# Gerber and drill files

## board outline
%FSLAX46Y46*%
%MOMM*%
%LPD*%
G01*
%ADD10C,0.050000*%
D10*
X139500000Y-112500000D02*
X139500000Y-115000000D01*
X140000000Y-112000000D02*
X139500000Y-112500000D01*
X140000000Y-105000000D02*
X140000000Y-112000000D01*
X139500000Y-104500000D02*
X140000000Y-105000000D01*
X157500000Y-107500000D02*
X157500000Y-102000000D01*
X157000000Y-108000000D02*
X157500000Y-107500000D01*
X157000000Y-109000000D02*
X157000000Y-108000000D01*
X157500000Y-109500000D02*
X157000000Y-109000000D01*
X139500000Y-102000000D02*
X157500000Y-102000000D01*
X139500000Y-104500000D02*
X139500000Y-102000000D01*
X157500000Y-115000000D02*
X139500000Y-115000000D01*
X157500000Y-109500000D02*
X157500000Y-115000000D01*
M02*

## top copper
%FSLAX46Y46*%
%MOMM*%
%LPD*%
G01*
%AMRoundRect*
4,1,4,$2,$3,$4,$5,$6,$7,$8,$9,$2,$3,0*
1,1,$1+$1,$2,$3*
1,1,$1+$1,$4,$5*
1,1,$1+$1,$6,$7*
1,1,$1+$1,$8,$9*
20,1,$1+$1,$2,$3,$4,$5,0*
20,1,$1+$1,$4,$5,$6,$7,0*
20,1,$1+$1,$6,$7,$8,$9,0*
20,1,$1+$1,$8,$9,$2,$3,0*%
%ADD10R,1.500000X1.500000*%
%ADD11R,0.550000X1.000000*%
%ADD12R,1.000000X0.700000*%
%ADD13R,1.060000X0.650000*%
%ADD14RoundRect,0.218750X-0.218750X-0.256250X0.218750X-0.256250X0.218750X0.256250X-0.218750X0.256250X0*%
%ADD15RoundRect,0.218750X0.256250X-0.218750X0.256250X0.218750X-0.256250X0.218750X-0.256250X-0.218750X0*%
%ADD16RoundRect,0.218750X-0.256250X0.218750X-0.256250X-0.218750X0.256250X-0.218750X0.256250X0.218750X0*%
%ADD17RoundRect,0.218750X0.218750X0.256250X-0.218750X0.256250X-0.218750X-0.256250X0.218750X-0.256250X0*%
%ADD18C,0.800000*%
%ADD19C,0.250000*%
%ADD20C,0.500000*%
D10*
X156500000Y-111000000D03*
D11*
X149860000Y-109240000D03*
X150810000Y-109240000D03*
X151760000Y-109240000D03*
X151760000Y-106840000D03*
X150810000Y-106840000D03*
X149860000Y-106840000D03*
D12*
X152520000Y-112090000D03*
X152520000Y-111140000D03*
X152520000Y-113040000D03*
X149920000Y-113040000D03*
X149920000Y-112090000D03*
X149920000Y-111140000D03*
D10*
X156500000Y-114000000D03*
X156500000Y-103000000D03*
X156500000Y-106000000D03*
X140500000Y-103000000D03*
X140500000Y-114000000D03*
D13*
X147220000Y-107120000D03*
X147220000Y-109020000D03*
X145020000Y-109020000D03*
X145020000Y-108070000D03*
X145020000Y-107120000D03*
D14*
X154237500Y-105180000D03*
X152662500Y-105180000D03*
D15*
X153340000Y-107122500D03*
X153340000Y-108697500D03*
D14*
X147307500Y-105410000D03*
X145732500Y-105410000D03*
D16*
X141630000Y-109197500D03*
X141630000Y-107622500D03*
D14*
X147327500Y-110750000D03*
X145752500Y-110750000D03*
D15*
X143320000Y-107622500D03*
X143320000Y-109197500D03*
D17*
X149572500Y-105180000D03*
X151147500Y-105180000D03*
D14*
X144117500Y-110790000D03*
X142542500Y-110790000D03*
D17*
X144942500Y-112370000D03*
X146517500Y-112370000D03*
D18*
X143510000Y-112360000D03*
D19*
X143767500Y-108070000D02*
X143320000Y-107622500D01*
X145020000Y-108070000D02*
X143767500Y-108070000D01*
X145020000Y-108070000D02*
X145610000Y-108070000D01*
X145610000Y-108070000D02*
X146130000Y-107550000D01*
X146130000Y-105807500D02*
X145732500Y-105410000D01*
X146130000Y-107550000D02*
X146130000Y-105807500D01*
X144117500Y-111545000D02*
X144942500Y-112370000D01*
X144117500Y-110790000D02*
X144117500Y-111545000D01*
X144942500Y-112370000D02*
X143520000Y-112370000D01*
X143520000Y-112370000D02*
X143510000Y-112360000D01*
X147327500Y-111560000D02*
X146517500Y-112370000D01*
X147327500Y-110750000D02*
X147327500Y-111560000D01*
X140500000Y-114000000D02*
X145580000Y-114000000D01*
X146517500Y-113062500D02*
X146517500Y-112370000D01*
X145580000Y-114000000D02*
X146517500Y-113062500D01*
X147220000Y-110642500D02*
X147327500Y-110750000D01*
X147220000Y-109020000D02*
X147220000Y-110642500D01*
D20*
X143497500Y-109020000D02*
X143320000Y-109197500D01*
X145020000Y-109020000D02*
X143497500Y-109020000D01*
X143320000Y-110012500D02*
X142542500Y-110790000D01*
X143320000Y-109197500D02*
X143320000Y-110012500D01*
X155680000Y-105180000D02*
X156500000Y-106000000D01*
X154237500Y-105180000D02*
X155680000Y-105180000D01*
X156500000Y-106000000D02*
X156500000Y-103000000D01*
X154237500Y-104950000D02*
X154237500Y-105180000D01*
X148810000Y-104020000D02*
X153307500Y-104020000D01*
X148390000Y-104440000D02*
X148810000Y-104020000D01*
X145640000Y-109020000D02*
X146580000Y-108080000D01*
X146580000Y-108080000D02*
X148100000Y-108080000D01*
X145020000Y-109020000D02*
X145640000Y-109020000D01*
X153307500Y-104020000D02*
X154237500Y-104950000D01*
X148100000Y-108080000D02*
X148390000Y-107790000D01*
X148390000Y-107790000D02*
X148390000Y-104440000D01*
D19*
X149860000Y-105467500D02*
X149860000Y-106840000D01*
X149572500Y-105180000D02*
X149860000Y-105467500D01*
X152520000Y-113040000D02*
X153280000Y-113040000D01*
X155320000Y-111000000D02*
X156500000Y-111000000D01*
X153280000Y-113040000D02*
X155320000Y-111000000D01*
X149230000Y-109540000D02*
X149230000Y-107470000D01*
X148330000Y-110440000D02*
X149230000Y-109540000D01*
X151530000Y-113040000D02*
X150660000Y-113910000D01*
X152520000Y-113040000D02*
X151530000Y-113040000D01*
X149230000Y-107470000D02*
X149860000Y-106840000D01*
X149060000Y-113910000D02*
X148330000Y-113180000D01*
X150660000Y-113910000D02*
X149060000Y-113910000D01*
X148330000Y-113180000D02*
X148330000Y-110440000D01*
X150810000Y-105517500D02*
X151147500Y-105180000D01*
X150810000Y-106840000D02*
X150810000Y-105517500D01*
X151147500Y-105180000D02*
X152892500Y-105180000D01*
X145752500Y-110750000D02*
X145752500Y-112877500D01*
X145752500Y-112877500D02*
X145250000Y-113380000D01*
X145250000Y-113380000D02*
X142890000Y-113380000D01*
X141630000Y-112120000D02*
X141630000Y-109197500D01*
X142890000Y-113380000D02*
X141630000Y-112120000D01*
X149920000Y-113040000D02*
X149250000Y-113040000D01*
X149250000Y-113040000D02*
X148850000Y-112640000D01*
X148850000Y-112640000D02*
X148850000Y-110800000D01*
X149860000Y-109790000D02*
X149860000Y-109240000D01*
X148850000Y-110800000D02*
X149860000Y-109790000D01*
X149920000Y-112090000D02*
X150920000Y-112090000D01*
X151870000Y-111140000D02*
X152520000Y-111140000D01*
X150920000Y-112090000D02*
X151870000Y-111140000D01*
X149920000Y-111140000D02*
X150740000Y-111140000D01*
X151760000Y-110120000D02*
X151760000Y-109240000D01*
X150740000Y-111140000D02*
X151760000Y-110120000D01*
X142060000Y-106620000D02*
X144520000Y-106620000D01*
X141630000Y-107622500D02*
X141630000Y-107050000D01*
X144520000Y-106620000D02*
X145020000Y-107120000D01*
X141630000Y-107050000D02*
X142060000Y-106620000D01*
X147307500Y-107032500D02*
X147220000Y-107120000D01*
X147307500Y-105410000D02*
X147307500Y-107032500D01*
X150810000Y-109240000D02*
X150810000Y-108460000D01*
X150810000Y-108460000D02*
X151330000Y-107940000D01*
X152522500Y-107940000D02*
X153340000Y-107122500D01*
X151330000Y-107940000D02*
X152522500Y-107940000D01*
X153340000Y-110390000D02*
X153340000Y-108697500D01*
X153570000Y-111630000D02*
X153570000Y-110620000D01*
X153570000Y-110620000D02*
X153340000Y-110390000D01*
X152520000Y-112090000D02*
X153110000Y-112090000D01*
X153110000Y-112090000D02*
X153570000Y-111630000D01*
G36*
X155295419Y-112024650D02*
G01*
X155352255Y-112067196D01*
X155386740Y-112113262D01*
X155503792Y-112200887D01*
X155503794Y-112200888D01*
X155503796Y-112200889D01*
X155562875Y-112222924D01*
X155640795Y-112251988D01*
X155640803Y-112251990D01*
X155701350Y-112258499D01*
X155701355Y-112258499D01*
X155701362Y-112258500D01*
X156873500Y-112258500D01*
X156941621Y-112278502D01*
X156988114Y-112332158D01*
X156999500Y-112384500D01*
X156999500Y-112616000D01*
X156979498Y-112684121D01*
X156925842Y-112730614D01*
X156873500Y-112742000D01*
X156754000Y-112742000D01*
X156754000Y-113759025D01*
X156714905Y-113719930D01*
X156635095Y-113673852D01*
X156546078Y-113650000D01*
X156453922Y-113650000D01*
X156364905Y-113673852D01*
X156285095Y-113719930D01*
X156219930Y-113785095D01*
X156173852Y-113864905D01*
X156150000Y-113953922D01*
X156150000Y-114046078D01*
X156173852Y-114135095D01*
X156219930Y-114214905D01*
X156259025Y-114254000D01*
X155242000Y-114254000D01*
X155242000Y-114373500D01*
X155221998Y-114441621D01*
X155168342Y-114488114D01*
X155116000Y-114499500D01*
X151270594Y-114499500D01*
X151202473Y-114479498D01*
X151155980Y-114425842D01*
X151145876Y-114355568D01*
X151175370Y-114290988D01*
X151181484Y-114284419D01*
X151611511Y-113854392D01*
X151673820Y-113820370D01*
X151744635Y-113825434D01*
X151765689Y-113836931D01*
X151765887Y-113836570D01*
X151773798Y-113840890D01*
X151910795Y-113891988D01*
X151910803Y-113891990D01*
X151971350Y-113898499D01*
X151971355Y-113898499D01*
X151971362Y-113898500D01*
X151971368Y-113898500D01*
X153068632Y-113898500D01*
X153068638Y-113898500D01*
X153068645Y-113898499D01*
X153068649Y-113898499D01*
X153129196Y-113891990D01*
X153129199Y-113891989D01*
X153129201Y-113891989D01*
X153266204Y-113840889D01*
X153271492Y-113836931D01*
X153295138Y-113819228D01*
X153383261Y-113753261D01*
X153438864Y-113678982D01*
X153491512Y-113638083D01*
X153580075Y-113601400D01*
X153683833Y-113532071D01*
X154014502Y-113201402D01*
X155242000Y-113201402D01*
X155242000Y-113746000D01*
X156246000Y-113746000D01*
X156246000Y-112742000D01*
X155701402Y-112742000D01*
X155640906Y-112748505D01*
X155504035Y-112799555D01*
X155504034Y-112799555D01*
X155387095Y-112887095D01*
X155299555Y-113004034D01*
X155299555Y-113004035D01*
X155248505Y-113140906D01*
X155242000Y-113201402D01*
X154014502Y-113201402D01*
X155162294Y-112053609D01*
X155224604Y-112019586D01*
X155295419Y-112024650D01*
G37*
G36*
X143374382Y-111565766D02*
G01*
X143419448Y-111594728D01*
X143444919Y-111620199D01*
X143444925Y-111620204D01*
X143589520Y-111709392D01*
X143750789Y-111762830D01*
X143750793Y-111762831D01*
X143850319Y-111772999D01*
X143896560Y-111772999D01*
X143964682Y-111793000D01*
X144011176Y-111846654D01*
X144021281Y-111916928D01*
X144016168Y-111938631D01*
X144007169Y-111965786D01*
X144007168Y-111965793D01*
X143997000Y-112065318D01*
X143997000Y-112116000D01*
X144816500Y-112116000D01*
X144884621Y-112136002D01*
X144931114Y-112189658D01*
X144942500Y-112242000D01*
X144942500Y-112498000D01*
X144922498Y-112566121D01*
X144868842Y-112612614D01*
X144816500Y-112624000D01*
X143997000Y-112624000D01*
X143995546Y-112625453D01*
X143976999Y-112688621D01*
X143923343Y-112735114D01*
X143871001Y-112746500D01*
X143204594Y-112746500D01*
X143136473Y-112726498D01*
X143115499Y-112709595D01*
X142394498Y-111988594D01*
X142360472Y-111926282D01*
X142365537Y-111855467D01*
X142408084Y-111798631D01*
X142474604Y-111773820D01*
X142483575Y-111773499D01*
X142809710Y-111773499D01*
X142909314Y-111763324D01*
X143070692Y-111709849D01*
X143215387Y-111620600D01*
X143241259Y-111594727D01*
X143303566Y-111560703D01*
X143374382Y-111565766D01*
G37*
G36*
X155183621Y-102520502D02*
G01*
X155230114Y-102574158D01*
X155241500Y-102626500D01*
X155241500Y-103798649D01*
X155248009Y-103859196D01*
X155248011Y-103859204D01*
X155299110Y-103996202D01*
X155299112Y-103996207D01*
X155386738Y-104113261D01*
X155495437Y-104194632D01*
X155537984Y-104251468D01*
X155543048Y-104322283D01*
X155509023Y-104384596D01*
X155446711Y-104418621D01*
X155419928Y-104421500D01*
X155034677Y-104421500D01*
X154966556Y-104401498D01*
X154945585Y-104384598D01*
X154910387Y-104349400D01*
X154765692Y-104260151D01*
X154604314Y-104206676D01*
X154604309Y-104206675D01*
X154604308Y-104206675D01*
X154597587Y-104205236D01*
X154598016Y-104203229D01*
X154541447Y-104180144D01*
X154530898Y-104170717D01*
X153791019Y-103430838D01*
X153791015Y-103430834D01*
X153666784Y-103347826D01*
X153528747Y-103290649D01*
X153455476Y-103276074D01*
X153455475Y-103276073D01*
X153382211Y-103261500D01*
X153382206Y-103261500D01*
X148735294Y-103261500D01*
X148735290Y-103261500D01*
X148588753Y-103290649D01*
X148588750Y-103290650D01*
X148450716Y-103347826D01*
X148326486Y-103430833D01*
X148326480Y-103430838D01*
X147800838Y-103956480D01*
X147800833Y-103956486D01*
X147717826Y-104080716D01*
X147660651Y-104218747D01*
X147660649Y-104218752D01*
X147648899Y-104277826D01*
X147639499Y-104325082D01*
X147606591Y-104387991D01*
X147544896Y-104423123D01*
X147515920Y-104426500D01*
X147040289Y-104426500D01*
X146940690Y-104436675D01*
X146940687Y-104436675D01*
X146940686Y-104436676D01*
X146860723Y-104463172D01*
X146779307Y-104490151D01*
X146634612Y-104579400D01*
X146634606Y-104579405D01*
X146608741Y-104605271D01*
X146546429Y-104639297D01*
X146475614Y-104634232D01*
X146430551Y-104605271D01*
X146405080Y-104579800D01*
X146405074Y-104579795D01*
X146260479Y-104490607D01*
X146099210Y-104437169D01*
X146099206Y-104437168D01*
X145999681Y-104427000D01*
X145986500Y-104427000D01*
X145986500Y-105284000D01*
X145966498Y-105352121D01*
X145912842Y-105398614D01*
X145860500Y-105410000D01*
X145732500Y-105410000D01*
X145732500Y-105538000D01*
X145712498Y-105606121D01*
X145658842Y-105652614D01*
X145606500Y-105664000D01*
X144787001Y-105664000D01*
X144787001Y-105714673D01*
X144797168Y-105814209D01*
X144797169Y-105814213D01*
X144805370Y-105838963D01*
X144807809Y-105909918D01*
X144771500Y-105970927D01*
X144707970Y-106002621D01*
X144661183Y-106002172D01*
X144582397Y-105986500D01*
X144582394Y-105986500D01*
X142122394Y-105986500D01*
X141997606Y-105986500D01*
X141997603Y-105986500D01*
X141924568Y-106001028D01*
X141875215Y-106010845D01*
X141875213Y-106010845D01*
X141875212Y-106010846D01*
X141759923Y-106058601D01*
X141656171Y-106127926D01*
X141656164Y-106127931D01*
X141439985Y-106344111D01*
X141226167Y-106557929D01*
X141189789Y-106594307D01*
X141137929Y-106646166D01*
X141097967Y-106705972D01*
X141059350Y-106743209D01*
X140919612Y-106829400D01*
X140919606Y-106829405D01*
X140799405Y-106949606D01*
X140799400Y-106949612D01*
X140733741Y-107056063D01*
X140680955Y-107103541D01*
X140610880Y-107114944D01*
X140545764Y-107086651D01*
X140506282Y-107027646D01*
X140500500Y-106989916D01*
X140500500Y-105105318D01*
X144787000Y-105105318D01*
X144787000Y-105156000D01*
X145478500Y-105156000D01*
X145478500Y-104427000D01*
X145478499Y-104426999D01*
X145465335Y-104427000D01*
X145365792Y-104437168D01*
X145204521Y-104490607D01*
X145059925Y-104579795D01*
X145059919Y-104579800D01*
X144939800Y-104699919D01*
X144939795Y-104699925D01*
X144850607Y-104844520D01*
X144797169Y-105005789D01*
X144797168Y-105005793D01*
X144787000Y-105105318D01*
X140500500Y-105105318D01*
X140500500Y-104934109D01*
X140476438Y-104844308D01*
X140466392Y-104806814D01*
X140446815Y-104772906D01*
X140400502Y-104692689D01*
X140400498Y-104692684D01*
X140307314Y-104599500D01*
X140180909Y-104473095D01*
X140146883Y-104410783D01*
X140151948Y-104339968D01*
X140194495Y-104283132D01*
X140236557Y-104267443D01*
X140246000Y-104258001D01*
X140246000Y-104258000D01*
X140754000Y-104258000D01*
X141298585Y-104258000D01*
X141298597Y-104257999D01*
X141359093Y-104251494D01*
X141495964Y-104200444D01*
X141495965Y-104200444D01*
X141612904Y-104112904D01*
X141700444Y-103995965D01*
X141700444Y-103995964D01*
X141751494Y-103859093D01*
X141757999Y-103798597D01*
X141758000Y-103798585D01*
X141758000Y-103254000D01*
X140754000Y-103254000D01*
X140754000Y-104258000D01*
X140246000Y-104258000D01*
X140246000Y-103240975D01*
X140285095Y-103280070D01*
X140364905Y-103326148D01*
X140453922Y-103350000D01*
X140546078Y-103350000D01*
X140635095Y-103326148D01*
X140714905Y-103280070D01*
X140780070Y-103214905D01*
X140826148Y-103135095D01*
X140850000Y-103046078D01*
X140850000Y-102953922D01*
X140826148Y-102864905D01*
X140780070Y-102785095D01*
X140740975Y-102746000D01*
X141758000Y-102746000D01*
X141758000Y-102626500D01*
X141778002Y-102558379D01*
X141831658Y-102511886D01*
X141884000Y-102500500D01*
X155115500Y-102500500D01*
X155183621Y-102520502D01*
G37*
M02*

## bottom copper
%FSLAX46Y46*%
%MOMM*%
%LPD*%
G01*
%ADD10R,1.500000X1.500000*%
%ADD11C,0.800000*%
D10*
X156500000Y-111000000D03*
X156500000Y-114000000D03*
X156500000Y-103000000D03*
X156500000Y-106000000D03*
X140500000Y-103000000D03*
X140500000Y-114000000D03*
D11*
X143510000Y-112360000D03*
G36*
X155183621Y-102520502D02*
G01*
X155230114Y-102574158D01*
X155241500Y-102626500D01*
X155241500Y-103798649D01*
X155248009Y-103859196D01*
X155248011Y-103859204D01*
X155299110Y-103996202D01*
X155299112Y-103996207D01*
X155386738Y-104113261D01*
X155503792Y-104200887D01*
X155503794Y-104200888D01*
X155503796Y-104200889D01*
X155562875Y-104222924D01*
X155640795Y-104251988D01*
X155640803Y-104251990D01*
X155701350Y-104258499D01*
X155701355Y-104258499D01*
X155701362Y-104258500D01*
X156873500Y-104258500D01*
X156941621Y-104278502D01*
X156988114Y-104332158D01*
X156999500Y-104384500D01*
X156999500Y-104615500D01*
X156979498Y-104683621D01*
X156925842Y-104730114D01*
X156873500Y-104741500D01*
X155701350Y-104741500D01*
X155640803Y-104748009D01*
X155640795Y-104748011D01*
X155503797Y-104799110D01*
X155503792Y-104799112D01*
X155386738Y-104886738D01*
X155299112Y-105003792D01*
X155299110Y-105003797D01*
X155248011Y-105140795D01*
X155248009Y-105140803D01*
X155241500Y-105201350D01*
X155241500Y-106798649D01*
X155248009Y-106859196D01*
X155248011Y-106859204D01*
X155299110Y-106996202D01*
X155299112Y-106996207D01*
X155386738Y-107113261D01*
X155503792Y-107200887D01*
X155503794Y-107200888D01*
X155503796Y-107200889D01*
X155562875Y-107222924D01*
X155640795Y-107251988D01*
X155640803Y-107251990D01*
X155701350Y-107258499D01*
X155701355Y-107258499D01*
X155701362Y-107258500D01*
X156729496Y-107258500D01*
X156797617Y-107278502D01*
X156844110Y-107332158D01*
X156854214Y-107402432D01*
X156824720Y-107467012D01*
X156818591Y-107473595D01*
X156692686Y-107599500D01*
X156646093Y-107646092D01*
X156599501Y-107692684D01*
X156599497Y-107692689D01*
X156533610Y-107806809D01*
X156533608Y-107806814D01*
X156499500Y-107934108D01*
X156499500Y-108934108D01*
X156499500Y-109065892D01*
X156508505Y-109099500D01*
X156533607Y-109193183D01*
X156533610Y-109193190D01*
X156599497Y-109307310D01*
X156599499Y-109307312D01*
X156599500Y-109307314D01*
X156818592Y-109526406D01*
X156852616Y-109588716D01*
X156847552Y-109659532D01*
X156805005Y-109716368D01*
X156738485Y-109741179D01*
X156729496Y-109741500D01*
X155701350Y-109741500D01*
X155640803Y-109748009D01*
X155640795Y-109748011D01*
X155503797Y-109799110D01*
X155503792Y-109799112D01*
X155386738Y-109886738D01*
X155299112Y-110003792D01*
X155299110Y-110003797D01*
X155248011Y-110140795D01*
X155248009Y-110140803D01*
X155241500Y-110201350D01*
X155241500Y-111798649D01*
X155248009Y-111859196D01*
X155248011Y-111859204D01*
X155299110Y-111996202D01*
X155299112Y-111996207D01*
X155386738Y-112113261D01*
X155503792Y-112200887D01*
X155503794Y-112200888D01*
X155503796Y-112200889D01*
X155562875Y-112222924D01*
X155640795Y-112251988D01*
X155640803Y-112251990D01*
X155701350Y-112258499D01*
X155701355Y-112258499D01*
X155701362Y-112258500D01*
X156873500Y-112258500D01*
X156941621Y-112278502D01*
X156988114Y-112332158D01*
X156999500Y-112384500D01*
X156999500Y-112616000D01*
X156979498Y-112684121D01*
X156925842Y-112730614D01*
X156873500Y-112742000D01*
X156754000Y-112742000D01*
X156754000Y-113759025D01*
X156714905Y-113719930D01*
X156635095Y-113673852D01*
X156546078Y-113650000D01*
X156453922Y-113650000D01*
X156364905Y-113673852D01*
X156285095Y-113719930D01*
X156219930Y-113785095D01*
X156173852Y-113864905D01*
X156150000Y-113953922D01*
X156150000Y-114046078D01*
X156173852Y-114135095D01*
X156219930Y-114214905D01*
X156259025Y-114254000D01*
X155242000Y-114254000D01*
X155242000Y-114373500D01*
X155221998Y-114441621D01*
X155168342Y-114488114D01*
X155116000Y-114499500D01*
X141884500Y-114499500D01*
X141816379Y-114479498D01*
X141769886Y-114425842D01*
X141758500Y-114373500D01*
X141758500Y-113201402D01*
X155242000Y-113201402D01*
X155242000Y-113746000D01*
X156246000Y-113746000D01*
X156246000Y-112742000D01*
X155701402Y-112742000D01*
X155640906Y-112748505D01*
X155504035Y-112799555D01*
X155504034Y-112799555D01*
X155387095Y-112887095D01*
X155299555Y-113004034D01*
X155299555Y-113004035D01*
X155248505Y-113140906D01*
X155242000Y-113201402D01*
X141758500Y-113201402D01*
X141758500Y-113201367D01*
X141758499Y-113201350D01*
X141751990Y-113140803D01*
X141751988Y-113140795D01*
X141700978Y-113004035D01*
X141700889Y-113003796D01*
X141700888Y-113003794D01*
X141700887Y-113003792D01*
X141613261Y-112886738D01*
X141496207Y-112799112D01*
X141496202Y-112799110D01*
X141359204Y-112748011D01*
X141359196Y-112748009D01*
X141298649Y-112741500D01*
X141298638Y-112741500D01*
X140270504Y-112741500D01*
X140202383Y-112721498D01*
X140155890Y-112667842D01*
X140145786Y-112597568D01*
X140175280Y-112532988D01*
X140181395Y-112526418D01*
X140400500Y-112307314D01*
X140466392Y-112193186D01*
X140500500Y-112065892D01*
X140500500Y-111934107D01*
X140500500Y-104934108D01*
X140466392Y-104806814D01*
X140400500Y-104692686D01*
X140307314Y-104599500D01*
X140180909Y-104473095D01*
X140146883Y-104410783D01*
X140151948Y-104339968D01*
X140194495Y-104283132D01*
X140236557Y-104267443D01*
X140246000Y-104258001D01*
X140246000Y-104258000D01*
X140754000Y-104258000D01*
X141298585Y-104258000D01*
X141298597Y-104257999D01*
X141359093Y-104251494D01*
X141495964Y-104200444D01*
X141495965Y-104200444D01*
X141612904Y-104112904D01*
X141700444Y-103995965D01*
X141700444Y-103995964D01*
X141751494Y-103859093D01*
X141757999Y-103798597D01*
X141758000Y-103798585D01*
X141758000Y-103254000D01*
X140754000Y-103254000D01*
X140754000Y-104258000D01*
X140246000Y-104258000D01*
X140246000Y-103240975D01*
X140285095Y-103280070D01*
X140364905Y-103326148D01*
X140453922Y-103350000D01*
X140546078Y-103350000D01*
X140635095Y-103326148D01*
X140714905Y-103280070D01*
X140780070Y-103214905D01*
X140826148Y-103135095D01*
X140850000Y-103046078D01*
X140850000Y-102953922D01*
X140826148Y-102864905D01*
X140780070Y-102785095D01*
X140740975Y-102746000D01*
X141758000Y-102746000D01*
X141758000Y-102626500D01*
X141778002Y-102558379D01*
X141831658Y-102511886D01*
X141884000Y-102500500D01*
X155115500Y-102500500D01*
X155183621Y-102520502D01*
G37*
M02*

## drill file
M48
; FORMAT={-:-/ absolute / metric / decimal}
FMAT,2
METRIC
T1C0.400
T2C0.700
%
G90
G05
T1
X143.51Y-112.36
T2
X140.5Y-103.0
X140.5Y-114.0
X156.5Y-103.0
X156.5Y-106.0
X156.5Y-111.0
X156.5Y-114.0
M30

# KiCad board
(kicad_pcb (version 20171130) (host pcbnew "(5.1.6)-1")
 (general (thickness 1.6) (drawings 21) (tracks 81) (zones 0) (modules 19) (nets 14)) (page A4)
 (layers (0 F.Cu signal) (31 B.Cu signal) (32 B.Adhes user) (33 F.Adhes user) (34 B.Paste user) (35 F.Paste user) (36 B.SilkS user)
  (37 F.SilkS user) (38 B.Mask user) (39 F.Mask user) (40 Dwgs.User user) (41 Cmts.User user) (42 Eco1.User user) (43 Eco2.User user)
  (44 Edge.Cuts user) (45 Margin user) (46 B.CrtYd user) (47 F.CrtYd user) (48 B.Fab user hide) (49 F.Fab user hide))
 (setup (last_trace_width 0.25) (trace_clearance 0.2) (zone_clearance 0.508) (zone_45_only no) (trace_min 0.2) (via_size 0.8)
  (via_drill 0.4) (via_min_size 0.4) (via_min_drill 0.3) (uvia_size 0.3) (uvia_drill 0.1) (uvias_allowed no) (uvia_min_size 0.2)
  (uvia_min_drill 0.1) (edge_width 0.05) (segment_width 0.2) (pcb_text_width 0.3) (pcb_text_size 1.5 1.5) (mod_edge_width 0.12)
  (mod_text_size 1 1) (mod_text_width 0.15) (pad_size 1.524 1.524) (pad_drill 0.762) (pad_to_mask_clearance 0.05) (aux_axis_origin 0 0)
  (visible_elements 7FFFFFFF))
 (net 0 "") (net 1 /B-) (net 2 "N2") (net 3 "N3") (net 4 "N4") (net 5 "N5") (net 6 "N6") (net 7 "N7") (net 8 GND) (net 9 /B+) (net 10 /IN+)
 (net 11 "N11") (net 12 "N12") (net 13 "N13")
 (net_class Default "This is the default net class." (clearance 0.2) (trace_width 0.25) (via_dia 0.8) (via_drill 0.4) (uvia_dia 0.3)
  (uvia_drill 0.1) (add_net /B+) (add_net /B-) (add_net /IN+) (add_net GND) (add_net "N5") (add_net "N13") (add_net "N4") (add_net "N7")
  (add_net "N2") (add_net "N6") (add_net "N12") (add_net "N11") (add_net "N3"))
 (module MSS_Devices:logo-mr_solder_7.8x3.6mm (layer B.Cu) (at 148.32 106.47 180)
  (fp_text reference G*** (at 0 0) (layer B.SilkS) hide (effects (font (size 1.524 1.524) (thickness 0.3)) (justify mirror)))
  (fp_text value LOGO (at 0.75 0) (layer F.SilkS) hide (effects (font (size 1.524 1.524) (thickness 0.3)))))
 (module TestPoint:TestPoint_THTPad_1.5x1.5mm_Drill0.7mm (layer F.Cu) (at 156.5 111)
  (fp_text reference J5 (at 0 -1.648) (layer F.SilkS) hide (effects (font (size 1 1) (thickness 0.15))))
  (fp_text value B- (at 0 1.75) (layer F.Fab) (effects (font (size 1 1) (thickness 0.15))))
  (pad 1 thru_hole rect (at 0 0) (size 1.5 1.5) (drill 0.7) (layers *.Cu *.Mask) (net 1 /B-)))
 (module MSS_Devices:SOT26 (layer F.Cu) (at 150.81 108.04)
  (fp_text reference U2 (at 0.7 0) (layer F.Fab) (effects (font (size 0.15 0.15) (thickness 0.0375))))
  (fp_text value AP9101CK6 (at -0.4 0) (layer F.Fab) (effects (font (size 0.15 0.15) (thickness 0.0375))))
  (pad 1 smd rect (at -0.95 1.2) (size 0.55 1) (layers F.Cu F.Paste F.Mask) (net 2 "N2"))
  (pad 2 smd rect (at 0 1.2) (size 0.55 1) (layers F.Cu F.Paste F.Mask) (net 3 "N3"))
  (pad 3 smd rect (at 0.95 1.2) (size 0.55 1) (layers F.Cu F.Paste F.Mask) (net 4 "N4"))
  (pad 4 smd rect (at 0.95 -1.2) (size 0.55 1) (layers F.Cu F.Paste F.Mask))
  (pad 5 smd rect (at 0 -1.2) (size 0.55 1) (layers F.Cu F.Paste F.Mask) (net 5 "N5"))
  (pad 6 smd rect (at -0.95 -1.2) (size 0.55 1) (layers F.Cu F.Paste F.Mask) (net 1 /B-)))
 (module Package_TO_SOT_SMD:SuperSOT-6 (layer F.Cu) (at 151.22 112.09)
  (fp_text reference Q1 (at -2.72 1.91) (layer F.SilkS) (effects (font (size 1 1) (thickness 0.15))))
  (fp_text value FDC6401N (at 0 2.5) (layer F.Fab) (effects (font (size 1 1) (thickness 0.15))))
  (pad 5 smd rect (at 1.3 0) (size 1 0.7) (layers F.Cu F.Paste F.Mask) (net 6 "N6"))
  (pad 6 smd rect (at 1.3 -0.95) (size 1 0.7) (layers F.Cu F.Paste F.Mask) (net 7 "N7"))
  (pad 4 smd rect (at 1.3 0.95) (size 1 0.7) (layers F.Cu F.Paste F.Mask) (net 1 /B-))
  (pad 3 smd rect (at -1.3 0.95) (size 1 0.7) (layers F.Cu F.Paste F.Mask) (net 2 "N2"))
  (pad 2 smd rect (at -1.3 0) (size 1 0.7) (layers F.Cu F.Paste F.Mask) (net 7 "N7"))
  (pad 1 smd rect (at -1.3 -0.95) (size 1 0.7) (layers F.Cu F.Paste F.Mask) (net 4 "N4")))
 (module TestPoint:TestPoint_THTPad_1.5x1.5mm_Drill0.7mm (layer F.Cu) (at 156.5 114)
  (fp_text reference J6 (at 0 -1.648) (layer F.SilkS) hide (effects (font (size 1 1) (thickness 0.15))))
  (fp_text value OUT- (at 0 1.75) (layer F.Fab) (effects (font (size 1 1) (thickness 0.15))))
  (pad 1 thru_hole rect (at 0 0) (size 1.5 1.5) (drill 0.7) (layers *.Cu *.Mask) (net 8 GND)))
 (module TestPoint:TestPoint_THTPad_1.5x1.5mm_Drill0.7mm (layer F.Cu) (at 156.5 103)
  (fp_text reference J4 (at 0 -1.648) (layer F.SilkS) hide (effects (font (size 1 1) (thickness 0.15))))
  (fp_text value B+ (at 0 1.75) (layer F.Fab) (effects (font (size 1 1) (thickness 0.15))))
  (pad 1 thru_hole rect (at 0 0) (size 1.5 1.5) (drill 0.7) (layers *.Cu *.Mask) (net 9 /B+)))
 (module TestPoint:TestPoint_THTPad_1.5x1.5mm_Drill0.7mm (layer F.Cu) (at 156.5 106)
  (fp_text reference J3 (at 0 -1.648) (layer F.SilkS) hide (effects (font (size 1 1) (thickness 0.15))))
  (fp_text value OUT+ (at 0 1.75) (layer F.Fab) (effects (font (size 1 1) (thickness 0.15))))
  (pad 1 thru_hole rect (at 0 0) (size 1.5 1.5) (drill 0.7) (layers *.Cu *.Mask) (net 9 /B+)))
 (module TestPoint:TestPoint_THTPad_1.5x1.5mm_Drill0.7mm (layer F.Cu) (at 140.5 103)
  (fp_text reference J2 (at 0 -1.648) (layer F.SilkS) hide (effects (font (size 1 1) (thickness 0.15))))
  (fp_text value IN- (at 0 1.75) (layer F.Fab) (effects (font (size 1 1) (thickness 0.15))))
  (pad 1 thru_hole rect (at 0 0) (size 1.5 1.5) (drill 0.7) (layers *.Cu *.Mask) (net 8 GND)))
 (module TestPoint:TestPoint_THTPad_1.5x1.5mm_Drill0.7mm (layer F.Cu) (at 140.5 114)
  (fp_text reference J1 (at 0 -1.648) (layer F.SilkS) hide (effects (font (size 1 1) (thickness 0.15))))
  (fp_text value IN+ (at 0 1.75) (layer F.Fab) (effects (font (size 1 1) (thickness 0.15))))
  (pad 1 thru_hole rect (at 0 0) (size 1.5 1.5) (drill 0.7) (layers *.Cu *.Mask) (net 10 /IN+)))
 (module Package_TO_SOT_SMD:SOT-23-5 (layer F.Cu) (at 146.12 108.07)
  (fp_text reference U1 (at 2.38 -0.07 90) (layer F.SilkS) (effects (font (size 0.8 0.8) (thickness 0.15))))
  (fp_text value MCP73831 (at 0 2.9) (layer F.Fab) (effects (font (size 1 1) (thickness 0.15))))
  (pad 5 smd rect (at 1.1 -0.95) (size 1.06 0.65) (layers F.Cu F.Paste F.Mask) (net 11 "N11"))
  (pad 4 smd rect (at 1.1 0.95) (size 1.06 0.65) (layers F.Cu F.Paste F.Mask) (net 10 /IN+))
  (pad 3 smd rect (at -1.1 0.95) (size 1.06 0.65) (layers F.Cu F.Paste F.Mask) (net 9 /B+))
  (pad 2 smd rect (at -1.1 0) (size 1.06 0.65) (layers F.Cu F.Paste F.Mask) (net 8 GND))
  (pad 1 smd rect (at -1.1 -0.95) (size 1.06 0.65) (layers F.Cu F.Paste F.Mask) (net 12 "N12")))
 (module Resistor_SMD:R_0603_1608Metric (layer F.Cu) (at 153.45 105.18)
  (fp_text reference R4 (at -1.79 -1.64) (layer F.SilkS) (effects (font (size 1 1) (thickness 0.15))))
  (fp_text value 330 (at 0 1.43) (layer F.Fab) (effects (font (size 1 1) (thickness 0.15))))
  (pad 2 smd roundrect (at 0.7875 0) (size 0.875 0.95) (layers F.Cu F.Paste F.Mask) (roundrect_rratio 0.25) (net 9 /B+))
  (pad 1 smd roundrect (at -0.7875 0) (size 0.875 0.95) (layers F.Cu F.Paste F.Mask) (roundrect_rratio 0.25) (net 5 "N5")))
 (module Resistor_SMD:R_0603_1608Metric (layer F.Cu) (at 153.34 107.91 90)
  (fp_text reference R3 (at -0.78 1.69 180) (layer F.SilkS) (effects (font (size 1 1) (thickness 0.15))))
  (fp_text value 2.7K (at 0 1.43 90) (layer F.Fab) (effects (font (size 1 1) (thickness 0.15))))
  (pad 2 smd roundrect (at 0.7875 0 90) (size 0.875 0.95) (layers F.Cu F.Paste F.Mask) (roundrect_rratio 0.25) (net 3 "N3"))
  (pad 1 smd roundrect (at -0.7875 0 90) (size 0.875 0.95) (layers F.Cu F.Paste F.Mask) (roundrect_rratio 0.25) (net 6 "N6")))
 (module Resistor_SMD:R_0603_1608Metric (layer F.Cu) (at 146.52 105.41)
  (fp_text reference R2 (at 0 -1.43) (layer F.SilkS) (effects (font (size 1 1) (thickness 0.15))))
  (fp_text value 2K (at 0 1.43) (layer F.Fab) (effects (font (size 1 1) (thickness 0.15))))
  (pad 2 smd roundrect (at 0.7875 0) (size 0.875 0.95) (layers F.Cu F.Paste F.Mask) (roundrect_rratio 0.25) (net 11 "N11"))
  (pad 1 smd roundrect (at -0.7875 0) (size 0.875 0.95) (layers F.Cu F.Paste F.Mask) (roundrect_rratio 0.25) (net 8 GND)))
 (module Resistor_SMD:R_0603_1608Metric (layer F.Cu) (at 141.63 108.41 270)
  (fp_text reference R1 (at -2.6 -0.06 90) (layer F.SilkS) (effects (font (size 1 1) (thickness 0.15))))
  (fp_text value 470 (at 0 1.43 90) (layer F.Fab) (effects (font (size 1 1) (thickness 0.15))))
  (pad 2 smd roundrect (at 0.7875 0 270) (size 0.875 0.95) (layers F.Cu F.Paste F.Mask) (roundrect_rratio 0.25) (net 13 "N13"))
  (pad 1 smd roundrect (at -0.7875 0 270) (size 0.875 0.95) (layers F.Cu F.Paste F.Mask) (roundrect_rratio 0.25) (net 12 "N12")))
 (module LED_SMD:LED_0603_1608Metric (layer F.Cu) (at 146.54 110.75)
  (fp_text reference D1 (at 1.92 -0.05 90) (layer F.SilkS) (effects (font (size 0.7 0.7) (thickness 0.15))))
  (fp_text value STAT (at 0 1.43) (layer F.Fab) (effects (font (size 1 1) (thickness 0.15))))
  (pad 2 smd roundrect (at 0.7875 0) (size 0.875 0.95) (layers F.Cu F.Paste F.Mask) (roundrect_rratio 0.25) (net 10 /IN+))
  (pad 1 smd roundrect (at -0.7875 0) (size 0.875 0.95) (layers F.Cu F.Paste F.Mask) (roundrect_rratio 0.25) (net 13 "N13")))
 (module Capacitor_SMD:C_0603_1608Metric (layer F.Cu) (at 143.32 108.41 90)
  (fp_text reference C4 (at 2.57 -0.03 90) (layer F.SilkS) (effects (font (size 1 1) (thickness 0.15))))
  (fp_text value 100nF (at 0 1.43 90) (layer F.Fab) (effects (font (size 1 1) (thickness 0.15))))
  (pad 2 smd roundrect (at 0.7875 0 90) (size 0.875 0.95) (layers F.Cu F.Paste F.Mask) (roundrect_rratio 0.25) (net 8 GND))
  (pad 1 smd roundrect (at -0.7875 0 90) (size 0.875 0.95) (layers F.Cu F.Paste F.Mask) (roundrect_rratio 0.25) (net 9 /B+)))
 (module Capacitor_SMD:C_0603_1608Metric (layer F.Cu) (at 150.36 105.18 180)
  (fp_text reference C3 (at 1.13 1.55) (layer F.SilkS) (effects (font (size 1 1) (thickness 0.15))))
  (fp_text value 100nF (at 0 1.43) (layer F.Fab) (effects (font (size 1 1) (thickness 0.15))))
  (pad 2 smd roundrect (at 0.7875 0 180) (size 0.875 0.95) (layers F.Cu F.Paste F.Mask) (roundrect_rratio 0.25) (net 1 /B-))
  (pad 1 smd roundrect (at -0.7875 0 180) (size 0.875 0.95) (layers F.Cu F.Paste F.Mask) (roundrect_rratio 0.25) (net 5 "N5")))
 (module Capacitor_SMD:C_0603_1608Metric (layer F.Cu) (at 143.33 110.79)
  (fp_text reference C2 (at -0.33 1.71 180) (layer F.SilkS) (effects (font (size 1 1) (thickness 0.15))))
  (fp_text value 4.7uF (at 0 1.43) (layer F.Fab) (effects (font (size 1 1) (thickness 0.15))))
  (pad 2 smd roundrect (at 0.7875 0) (size 0.875 0.95) (layers F.Cu F.Paste F.Mask) (roundrect_rratio 0.25) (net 8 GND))
  (pad 1 smd roundrect (at -0.7875 0) (size 0.875 0.95) (layers F.Cu F.Paste F.Mask) (roundrect_rratio 0.25) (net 9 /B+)))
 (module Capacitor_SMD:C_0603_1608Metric (layer F.Cu) (at 145.73 112.37 180)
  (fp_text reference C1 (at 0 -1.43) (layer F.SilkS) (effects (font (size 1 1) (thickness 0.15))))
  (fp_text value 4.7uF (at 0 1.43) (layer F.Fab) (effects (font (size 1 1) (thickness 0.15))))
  (pad 2 smd roundrect (at 0.7875 0 180) (size 0.875 0.95) (layers F.Cu F.Paste F.Mask) (roundrect_rratio 0.25) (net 8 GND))
  (pad 1 smd roundrect (at -0.7875 0 180) (size 0.875 0.95) (layers F.Cu F.Paste F.Mask) (roundrect_rratio 0.25) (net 10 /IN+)))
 (gr_line (start 139.5 112.5) (end 139.5 115) (layer Edge.Cuts) (width 0.05))
 (gr_line (start 140 112) (end 139.5 112.5) (layer Edge.Cuts) (width 0.05))
 (gr_line (start 140 105) (end 140 112) (layer Edge.Cuts) (width 0.05))
 (gr_line (start 139.5 104.5) (end 140 105) (layer Edge.Cuts) (width 0.05))
 (gr_line (start 157.5 107.5) (end 157.5 102) (layer Edge.Cuts) (width 0.05))
 (gr_line (start 157 108) (end 157.5 107.5) (layer Edge.Cuts) (width 0.05))
 (gr_line (start 157 109) (end 157 108) (layer Edge.Cuts) (width 0.05))
 (gr_line (start 157.5 109.5) (end 157 109) (layer Edge.Cuts) (width 0.05))
 (gr_line (start 139.5 102) (end 157.5 102) (layer Edge.Cuts) (width 0.05))
 (gr_line (start 139.5 104.5) (end 139.5 102) (layer Edge.Cuts) (width 0.05))
 (gr_line (start 157.5 115) (end 139.5 115) (layer Edge.Cuts) (width 0.05))
 (gr_line (start 157.5 109.5) (end 157.5 115) (layer Edge.Cuts) (width 0.05))
 (segment (start 143.7675 108.07) (end 143.32 107.6225) (width 0.25) (layer F.Cu) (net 8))
 (segment (start 145.02 108.07) (end 143.7675 108.07) (width 0.25) (layer F.Cu) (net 8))
 (segment (start 145.02 108.07) (end 145.61 108.07) (width 0.25) (layer F.Cu) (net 8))
 (segment (start 145.61 108.07) (end 146.13 107.55) (width 0.25) (layer F.Cu) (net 8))
 (segment (start 146.13 105.8075) (end 145.7325 105.41) (width 0.25) (layer F.Cu) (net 8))
 (segment (start 146.13 107.55) (end 146.13 105.8075) (width 0.25) (layer F.Cu) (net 8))
 (segment (start 144.1175 111.545) (end 144.9425 112.37) (width 0.25) (layer F.Cu) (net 8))
 (segment (start 144.1175 110.79) (end 144.1175 111.545) (width 0.25) (layer F.Cu) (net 8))
 (via (at 143.51 112.36) (size 0.8) (drill 0.4) (layers F.Cu B.Cu) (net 8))
 (segment (start 144.9425 112.37) (end 143.52 112.37) (width 0.25) (layer F.Cu) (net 8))
 (segment (start 143.52 112.37) (end 143.51 112.36) (width 0.25) (layer F.Cu) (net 8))
 (segment (start 147.3275 111.56) (end 146.5175 112.37) (width 0.25) (layer F.Cu) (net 10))
 (segment (start 147.3275 110.75) (end 147.3275 111.56) (width 0.25) (layer F.Cu) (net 10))
 (segment (start 140.5 114) (end 145.58 114) (width 0.25) (layer F.Cu) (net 10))
 (segment (start 146.5175 113.0625) (end 146.5175 112.37) (width 0.25) (layer F.Cu) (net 10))
 (segment (start 145.58 114) (end 146.5175 113.0625) (width 0.25) (layer F.Cu) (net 10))
 (segment (start 147.22 110.6425) (end 147.3275 110.75) (width 0.25) (layer F.Cu) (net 10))
 (segment (start 147.22 109.02) (end 147.22 110.6425) (width 0.25) (layer F.Cu) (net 10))
 (segment (start 143.4975 109.02) (end 143.32 109.1975) (width 0.5) (layer F.Cu) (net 9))
 (segment (start 145.02 109.02) (end 143.4975 109.02) (width 0.5) (layer F.Cu) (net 9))
 (segment (start 143.32 110.0125) (end 142.5425 110.79) (width 0.5) (layer F.Cu) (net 9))
 (segment (start 143.32 109.1975) (end 143.32 110.0125) (width 0.5) (layer F.Cu) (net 9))
 (segment (start 155.68 105.18) (end 156.5 106) (width 0.5) (layer F.Cu) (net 9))
 (segment (start 154.2375 105.18) (end 155.68 105.18) (width 0.5) (layer F.Cu) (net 9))
 (segment (start 156.5 106) (end 156.5 103) (width 0.5) (layer F.Cu) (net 9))
 (segment (start 154.2375 104.95) (end 154.2375 105.18) (width 0.5) (layer F.Cu) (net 9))
 (segment (start 148.81 104.02) (end 153.3075 104.02) (width 0.5) (layer F.Cu) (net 9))
 (segment (start 148.39 104.44) (end 148.81 104.02) (width 0.5) (layer F.Cu) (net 9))
 (segment (start 145.64 109.02) (end 146.58 108.08) (width 0.5) (layer F.Cu) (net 9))
 (segment (start 146.58 108.08) (end 148.1 108.08) (width 0.5) (layer F.Cu) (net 9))
 (segment (start 145.02 109.02) (end 145.64 109.02) (width 0.5) (layer F.Cu) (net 9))
 (segment (start 153.3075 104.02) (end 154.2375 104.95) (width 0.5) (layer F.Cu) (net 9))
 (segment (start 148.1 108.08) (end 148.39 107.79) (width 0.5) (layer F.Cu) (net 9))
 (segment (start 148.39 107.79) (end 148.39 104.44) (width 0.5) (layer F.Cu) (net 9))
 (segment (start 149.86 105.4675) (end 149.86 106.84) (width 0.25) (layer F.Cu) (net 1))
 (segment (start 149.5725 105.18) (end 149.86 105.4675) (width 0.25) (layer F.Cu) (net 1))
 (segment (start 152.52 113.04) (end 153.28 113.04) (width 0.25) (layer F.Cu) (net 1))
 (segment (start 155.32 111) (end 156.5 111) (width 0.25) (layer F.Cu) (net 1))
 (segment (start 153.28 113.04) (end 155.32 111) (width 0.25) (layer F.Cu) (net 1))
 (segment (start 149.23 109.54) (end 149.23 107.47) (width 0.25) (layer F.Cu) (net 1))
 (segment (start 148.33 110.44) (end 149.23 109.54) (width 0.25) (layer F.Cu) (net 1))
 (segment (start 151.53 113.04) (end 150.66 113.91) (width 0.25) (layer F.Cu) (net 1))
 (segment (start 152.52 113.04) (end 151.53 113.04) (width 0.25) (layer F.Cu) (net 1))
 (segment (start 149.23 107.47) (end 149.86 106.84) (width 0.25) (layer F.Cu) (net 1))
 (segment (start 149.06 113.91) (end 148.33 113.18) (width 0.25) (layer F.Cu) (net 1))
 (segment (start 150.66 113.91) (end 149.06 113.91) (width 0.25) (layer F.Cu) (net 1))
 (segment (start 148.33 113.18) (end 148.33 110.44) (width 0.25) (layer F.Cu) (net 1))
 (segment (start 150.81 105.5175) (end 151.1475 105.18) (width 0.25) (layer F.Cu) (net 5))
 (segment (start 150.81 106.84) (end 150.81 105.5175) (width 0.25) (layer F.Cu) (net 5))
 (segment (start 151.1475 105.18) (end 152.8925 105.18) (width 0.25) (layer F.Cu) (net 5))
 (segment (start 145.7525 110.75) (end 145.7525 112.8775) (width 0.25) (layer F.Cu) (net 13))
 (segment (start 145.7525 112.8775) (end 145.25 113.38) (width 0.25) (layer F.Cu) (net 13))
 (segment (start 145.25 113.38) (end 142.89 113.38) (width 0.25) (layer F.Cu) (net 13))
 (segment (start 141.63 112.12) (end 141.63 109.1975) (width 0.25) (layer F.Cu) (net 13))
 (segment (start 142.89 113.38) (end 141.63 112.12) (width 0.25) (layer F.Cu) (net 13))
 (segment (start 149.92 113.04) (end 149.25 113.04) (width 0.25) (layer F.Cu) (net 2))
 (segment (start 149.25 113.04) (end 148.85 112.64) (width 0.25) (layer F.Cu) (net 2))
 (segment (start 148.85 112.64) (end 148.85 110.8) (width 0.25) (layer F.Cu) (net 2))
 (segment (start 149.86 109.79) (end 149.86 109.24) (width 0.25) (layer F.Cu) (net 2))
 (segment (start 148.85 110.8) (end 149.86 109.79) (width 0.25) (layer F.Cu) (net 2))
 (segment (start 149.92 112.09) (end 150.92 112.09) (width 0.25) (layer F.Cu) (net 7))
 (segment (start 151.87 111.14) (end 152.52 111.14) (width 0.25) (layer F.Cu) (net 7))
 (segment (start 150.92 112.09) (end 151.87 111.14) (width 0.25) (layer F.Cu) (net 7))
 (segment (start 149.92 111.14) (end 150.74 111.14) (width 0.25) (layer F.Cu) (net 4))
 (segment (start 151.76 110.12) (end 151.76 109.24) (width 0.25) (layer F.Cu) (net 4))
 (segment (start 150.74 111.14) (end 151.76 110.12) (width 0.25) (layer F.Cu) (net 4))
 (segment (start 142.06 106.62) (end 144.52 106.62) (width 0.25) (layer F.Cu) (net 12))
 (segment (start 141.63 107.6225) (end 141.63 107.05) (width 0.25) (layer F.Cu) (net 12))
 (segment (start 144.52 106.62) (end 145.02 107.12) (width 0.25) (layer F.Cu) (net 12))
 (segment (start 141.63 107.05) (end 142.06 106.62) (width 0.25) (layer F.Cu) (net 12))
 (segment (start 147.3075 107.0325) (end 147.22 107.12) (width 0.25) (layer F.Cu) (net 11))
 (segment (start 147.3075 105.41) (end 147.3075 107.0325) (width 0.25) (layer F.Cu) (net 11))
 (segment (start 150.81 109.24) (end 150.81 108.46) (width 0.25) (layer F.Cu) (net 3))
 (segment (start 150.81 108.46) (end 151.33 107.94) (width 0.25) (layer F.Cu) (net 3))
 (segment (start 152.5225 107.94) (end 153.34 107.1225) (width 0.25) (layer F.Cu) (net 3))
 (segment (start 151.33 107.94) (end 152.5225 107.94) (width 0.25) (layer F.Cu) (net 3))
 (segment (start 153.34 110.39) (end 153.34 108.6975) (width 0.25) (layer F.Cu) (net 6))
 (segment (start 153.57 111.63) (end 153.57 110.62) (width 0.25) (layer F.Cu) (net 6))
 (segment (start 153.57 110.62) (end 153.34 110.39) (width 0.25) (layer F.Cu) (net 6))
 (segment (start 152.52 112.09) (end 153.11 112.09) (width 0.25) (layer F.Cu) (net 6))
 (segment (start 153.11 112.09) (end 153.57 111.63) (width 0.25) (layer F.Cu) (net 6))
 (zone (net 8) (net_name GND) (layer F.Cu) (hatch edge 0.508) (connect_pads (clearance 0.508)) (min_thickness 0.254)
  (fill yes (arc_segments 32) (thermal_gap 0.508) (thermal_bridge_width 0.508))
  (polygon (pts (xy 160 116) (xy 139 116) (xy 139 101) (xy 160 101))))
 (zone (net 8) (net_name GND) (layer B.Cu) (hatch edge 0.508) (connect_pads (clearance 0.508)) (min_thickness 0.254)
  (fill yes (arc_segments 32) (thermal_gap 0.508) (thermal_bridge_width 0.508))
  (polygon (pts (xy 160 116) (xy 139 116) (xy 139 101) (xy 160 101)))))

